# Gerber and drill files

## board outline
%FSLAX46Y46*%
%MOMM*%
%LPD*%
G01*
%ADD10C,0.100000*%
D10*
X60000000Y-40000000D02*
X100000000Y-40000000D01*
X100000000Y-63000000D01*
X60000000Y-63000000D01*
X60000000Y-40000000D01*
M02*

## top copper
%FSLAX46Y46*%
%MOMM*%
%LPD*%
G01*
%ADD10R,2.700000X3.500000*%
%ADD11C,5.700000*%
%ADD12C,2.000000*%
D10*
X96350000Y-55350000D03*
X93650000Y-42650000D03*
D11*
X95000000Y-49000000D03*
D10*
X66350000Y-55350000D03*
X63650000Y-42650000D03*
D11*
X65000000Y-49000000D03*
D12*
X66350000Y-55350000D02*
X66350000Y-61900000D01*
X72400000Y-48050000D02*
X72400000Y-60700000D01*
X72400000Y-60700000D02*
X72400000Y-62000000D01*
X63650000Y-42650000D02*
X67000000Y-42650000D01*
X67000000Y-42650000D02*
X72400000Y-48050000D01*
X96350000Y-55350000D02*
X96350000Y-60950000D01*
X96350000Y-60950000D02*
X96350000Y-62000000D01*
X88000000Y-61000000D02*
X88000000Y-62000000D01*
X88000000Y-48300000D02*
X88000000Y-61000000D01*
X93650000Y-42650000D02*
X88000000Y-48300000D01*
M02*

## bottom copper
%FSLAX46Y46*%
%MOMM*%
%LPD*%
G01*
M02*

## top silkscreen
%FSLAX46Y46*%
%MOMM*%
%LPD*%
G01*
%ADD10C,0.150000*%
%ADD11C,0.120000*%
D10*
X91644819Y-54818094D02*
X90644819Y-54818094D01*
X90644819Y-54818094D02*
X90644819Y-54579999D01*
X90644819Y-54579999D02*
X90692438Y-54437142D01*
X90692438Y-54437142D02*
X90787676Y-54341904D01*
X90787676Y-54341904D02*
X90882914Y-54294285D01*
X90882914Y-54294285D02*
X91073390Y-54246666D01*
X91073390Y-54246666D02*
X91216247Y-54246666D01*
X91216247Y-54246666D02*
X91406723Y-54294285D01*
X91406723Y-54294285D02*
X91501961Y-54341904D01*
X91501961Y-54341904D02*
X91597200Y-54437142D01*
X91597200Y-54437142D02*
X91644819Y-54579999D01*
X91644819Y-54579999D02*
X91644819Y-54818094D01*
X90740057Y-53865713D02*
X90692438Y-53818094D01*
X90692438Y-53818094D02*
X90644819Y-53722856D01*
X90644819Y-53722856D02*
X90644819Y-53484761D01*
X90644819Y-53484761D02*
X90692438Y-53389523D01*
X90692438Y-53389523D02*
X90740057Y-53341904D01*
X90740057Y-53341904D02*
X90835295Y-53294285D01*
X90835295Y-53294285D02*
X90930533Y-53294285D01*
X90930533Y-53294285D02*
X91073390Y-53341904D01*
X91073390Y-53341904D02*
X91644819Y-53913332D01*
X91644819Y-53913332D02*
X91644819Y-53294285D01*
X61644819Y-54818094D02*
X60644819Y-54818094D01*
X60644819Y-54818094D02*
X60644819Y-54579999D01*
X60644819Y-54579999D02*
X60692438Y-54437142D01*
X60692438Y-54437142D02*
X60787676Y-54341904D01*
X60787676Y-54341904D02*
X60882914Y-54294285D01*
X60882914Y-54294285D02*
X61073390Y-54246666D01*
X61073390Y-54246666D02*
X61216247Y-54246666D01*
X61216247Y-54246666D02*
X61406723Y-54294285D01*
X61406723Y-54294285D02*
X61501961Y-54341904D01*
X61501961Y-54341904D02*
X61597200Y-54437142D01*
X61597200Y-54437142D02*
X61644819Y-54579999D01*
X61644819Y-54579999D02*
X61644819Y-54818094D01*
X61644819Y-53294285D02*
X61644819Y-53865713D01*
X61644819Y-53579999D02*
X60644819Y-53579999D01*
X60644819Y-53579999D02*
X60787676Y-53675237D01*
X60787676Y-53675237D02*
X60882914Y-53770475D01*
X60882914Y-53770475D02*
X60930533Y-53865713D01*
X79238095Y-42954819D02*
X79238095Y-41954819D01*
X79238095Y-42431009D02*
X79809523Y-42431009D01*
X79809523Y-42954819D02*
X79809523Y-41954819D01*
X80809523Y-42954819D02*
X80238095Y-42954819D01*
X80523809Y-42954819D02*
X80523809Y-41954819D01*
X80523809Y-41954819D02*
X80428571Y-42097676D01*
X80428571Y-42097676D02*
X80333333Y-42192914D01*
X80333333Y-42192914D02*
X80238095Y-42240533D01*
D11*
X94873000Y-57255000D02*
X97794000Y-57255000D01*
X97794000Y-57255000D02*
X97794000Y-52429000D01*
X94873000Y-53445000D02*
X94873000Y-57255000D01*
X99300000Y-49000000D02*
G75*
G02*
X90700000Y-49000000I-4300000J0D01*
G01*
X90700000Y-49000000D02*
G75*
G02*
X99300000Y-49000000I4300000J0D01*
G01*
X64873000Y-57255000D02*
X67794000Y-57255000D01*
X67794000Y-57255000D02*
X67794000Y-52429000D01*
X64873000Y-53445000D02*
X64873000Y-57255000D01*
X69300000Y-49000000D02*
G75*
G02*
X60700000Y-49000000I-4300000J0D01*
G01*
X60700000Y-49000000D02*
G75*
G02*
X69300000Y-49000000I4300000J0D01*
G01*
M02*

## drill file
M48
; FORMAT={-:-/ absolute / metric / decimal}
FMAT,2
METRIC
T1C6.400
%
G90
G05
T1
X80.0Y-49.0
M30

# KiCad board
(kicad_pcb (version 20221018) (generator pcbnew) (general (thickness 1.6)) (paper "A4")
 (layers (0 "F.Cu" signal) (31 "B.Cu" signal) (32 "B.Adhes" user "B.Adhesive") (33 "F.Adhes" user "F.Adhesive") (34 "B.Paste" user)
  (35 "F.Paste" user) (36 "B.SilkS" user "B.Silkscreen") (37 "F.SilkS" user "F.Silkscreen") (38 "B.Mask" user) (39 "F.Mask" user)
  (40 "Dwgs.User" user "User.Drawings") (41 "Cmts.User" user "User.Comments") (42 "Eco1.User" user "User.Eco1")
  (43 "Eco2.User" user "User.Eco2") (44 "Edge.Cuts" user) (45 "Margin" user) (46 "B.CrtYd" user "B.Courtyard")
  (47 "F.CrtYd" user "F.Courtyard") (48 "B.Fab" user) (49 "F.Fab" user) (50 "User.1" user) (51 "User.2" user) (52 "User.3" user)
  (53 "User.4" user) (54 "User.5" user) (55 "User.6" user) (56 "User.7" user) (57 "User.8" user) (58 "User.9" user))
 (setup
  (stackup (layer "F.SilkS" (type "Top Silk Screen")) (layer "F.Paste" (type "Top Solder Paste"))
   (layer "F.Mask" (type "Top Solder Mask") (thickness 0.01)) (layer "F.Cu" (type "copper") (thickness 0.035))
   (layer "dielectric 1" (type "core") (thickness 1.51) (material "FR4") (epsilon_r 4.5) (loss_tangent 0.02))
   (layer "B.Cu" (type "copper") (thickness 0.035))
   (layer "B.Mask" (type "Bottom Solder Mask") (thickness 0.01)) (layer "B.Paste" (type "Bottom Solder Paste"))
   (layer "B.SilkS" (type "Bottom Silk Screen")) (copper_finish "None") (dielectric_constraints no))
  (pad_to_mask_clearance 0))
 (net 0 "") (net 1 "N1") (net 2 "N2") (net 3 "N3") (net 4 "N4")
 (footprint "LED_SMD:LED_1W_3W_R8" (layer "F.Cu") (at 95 49 90)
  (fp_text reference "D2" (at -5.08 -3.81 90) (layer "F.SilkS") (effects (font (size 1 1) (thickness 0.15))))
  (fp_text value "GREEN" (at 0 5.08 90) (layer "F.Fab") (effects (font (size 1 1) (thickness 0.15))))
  (fp_line (start -8.255 -0.127) (end -8.255 2.794) (stroke (width 0.12) (type solid)) (layer "F.SilkS"))
  (fp_line (start -8.255 2.794) (end -3.429 2.794) (stroke (width 0.12) (type solid)) (layer "F.SilkS"))
  (fp_line (start -4.445 -0.127) (end -8.255 -0.127) (stroke (width 0.12) (type solid)) (layer "F.SilkS"))
  (fp_circle (center 0 0) (end -4.3 0) (stroke (width 0.12) (type solid)) (fill none) (layer "F.SilkS"))
  (pad "1" smd rect (at -6.35 1.35 90) (size 3.5 2.7) (layers "F.Cu" "F.Paste" "F.Mask") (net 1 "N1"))
  (pad "2" smd rect (at 6.35 -1.35 90) (size 3.5 2.7) (layers "F.Cu" "F.Paste" "F.Mask") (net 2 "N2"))
  (pad "3" smd circle (at 0 0 90) (size 5.7 5.7) (layers "F.Cu" "F.Paste" "F.Mask")))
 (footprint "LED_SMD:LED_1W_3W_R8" (layer "F.Cu") (at 65 49 90)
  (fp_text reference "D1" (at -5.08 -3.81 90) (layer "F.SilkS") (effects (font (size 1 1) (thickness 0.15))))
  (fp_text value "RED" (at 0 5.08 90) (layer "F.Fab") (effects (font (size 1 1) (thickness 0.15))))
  (fp_line (start -8.255 -0.127) (end -8.255 2.794) (stroke (width 0.12) (type solid)) (layer "F.SilkS"))
  (fp_line (start -8.255 2.794) (end -3.429 2.794) (stroke (width 0.12) (type solid)) (layer "F.SilkS"))
  (fp_line (start -4.445 -0.127) (end -8.255 -0.127) (stroke (width 0.12) (type solid)) (layer "F.SilkS"))
  (fp_circle (center 0 0) (end -4.3 0) (stroke (width 0.12) (type solid)) (fill none) (layer "F.SilkS"))
  (pad "1" smd rect (at -6.35 1.35 90) (size 3.5 2.7) (layers "F.Cu" "F.Paste" "F.Mask") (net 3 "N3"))
  (pad "2" smd rect (at 6.35 -1.35 90) (size 3.5 2.7) (layers "F.Cu" "F.Paste" "F.Mask") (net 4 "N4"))
  (pad "3" smd circle (at 0 0 90) (size 5.7 5.7) (layers "F.Cu" "F.Paste" "F.Mask")))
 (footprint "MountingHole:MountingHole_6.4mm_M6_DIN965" (layer "F.Cu") (at 80 49)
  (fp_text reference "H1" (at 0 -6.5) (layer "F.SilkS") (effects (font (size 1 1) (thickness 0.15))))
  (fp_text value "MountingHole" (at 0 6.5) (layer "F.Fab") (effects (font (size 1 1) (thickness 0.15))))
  (pad "" np_thru_hole circle (at 0 0) (size 6.4 6.4) (drill 6.4) (layers "*.Cu" "*.Mask")))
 (gr_rect (start 60 40) (end 100 63) (stroke (width 0.1) (type default)) (fill none) (layer "Edge.Cuts"))
 (segment (start 66.35 55.35) (end 66.35 61.9) (width 2) (layer "F.Cu") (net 3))
 (segment (start 72.4 48.05) (end 72.4 60.7) (width 2) (layer "F.Cu") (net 4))
 (segment (start 72.4 60.7) (end 72.4 62) (width 2) (layer "F.Cu") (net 4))
 (segment (start 63.65 42.65) (end 67 42.65) (width 2) (layer "F.Cu") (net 4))
 (segment (start 67 42.65) (end 72.4 48.05) (width 2) (layer "F.Cu") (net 4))
 (segment (start 96.35 55.35) (end 96.35 60.95) (width 2) (layer "F.Cu") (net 1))
 (segment (start 96.35 60.95) (end 96.35 62) (width 2) (layer "F.Cu") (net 1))
 (segment (start 88 61) (end 88 62) (width 2) (layer "F.Cu") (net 2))
 (segment (start 88 48.3) (end 88 61) (width 2) (layer "F.Cu") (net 2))
 (segment (start 93.65 42.65) (end 88 48.3) (width 2) (layer "F.Cu") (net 2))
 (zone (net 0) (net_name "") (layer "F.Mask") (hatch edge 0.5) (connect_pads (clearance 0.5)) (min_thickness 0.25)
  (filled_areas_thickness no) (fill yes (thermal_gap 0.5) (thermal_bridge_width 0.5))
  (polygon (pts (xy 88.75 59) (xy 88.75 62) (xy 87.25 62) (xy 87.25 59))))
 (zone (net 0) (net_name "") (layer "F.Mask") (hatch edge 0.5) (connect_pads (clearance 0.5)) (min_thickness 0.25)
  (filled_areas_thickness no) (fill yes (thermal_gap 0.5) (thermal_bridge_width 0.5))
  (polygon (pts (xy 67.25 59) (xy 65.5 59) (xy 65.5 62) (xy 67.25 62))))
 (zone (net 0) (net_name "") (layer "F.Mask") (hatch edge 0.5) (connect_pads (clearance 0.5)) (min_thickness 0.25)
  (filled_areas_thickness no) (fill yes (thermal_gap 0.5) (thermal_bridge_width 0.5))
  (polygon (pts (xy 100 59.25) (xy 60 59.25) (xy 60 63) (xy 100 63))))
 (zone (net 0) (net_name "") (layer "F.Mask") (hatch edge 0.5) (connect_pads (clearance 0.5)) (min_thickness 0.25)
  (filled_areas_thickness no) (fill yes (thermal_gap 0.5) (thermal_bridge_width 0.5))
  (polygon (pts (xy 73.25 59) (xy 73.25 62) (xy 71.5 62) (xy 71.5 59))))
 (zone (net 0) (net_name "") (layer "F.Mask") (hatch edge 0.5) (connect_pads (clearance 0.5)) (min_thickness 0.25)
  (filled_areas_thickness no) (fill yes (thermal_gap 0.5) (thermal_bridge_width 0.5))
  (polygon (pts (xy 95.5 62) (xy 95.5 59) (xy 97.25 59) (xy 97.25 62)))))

